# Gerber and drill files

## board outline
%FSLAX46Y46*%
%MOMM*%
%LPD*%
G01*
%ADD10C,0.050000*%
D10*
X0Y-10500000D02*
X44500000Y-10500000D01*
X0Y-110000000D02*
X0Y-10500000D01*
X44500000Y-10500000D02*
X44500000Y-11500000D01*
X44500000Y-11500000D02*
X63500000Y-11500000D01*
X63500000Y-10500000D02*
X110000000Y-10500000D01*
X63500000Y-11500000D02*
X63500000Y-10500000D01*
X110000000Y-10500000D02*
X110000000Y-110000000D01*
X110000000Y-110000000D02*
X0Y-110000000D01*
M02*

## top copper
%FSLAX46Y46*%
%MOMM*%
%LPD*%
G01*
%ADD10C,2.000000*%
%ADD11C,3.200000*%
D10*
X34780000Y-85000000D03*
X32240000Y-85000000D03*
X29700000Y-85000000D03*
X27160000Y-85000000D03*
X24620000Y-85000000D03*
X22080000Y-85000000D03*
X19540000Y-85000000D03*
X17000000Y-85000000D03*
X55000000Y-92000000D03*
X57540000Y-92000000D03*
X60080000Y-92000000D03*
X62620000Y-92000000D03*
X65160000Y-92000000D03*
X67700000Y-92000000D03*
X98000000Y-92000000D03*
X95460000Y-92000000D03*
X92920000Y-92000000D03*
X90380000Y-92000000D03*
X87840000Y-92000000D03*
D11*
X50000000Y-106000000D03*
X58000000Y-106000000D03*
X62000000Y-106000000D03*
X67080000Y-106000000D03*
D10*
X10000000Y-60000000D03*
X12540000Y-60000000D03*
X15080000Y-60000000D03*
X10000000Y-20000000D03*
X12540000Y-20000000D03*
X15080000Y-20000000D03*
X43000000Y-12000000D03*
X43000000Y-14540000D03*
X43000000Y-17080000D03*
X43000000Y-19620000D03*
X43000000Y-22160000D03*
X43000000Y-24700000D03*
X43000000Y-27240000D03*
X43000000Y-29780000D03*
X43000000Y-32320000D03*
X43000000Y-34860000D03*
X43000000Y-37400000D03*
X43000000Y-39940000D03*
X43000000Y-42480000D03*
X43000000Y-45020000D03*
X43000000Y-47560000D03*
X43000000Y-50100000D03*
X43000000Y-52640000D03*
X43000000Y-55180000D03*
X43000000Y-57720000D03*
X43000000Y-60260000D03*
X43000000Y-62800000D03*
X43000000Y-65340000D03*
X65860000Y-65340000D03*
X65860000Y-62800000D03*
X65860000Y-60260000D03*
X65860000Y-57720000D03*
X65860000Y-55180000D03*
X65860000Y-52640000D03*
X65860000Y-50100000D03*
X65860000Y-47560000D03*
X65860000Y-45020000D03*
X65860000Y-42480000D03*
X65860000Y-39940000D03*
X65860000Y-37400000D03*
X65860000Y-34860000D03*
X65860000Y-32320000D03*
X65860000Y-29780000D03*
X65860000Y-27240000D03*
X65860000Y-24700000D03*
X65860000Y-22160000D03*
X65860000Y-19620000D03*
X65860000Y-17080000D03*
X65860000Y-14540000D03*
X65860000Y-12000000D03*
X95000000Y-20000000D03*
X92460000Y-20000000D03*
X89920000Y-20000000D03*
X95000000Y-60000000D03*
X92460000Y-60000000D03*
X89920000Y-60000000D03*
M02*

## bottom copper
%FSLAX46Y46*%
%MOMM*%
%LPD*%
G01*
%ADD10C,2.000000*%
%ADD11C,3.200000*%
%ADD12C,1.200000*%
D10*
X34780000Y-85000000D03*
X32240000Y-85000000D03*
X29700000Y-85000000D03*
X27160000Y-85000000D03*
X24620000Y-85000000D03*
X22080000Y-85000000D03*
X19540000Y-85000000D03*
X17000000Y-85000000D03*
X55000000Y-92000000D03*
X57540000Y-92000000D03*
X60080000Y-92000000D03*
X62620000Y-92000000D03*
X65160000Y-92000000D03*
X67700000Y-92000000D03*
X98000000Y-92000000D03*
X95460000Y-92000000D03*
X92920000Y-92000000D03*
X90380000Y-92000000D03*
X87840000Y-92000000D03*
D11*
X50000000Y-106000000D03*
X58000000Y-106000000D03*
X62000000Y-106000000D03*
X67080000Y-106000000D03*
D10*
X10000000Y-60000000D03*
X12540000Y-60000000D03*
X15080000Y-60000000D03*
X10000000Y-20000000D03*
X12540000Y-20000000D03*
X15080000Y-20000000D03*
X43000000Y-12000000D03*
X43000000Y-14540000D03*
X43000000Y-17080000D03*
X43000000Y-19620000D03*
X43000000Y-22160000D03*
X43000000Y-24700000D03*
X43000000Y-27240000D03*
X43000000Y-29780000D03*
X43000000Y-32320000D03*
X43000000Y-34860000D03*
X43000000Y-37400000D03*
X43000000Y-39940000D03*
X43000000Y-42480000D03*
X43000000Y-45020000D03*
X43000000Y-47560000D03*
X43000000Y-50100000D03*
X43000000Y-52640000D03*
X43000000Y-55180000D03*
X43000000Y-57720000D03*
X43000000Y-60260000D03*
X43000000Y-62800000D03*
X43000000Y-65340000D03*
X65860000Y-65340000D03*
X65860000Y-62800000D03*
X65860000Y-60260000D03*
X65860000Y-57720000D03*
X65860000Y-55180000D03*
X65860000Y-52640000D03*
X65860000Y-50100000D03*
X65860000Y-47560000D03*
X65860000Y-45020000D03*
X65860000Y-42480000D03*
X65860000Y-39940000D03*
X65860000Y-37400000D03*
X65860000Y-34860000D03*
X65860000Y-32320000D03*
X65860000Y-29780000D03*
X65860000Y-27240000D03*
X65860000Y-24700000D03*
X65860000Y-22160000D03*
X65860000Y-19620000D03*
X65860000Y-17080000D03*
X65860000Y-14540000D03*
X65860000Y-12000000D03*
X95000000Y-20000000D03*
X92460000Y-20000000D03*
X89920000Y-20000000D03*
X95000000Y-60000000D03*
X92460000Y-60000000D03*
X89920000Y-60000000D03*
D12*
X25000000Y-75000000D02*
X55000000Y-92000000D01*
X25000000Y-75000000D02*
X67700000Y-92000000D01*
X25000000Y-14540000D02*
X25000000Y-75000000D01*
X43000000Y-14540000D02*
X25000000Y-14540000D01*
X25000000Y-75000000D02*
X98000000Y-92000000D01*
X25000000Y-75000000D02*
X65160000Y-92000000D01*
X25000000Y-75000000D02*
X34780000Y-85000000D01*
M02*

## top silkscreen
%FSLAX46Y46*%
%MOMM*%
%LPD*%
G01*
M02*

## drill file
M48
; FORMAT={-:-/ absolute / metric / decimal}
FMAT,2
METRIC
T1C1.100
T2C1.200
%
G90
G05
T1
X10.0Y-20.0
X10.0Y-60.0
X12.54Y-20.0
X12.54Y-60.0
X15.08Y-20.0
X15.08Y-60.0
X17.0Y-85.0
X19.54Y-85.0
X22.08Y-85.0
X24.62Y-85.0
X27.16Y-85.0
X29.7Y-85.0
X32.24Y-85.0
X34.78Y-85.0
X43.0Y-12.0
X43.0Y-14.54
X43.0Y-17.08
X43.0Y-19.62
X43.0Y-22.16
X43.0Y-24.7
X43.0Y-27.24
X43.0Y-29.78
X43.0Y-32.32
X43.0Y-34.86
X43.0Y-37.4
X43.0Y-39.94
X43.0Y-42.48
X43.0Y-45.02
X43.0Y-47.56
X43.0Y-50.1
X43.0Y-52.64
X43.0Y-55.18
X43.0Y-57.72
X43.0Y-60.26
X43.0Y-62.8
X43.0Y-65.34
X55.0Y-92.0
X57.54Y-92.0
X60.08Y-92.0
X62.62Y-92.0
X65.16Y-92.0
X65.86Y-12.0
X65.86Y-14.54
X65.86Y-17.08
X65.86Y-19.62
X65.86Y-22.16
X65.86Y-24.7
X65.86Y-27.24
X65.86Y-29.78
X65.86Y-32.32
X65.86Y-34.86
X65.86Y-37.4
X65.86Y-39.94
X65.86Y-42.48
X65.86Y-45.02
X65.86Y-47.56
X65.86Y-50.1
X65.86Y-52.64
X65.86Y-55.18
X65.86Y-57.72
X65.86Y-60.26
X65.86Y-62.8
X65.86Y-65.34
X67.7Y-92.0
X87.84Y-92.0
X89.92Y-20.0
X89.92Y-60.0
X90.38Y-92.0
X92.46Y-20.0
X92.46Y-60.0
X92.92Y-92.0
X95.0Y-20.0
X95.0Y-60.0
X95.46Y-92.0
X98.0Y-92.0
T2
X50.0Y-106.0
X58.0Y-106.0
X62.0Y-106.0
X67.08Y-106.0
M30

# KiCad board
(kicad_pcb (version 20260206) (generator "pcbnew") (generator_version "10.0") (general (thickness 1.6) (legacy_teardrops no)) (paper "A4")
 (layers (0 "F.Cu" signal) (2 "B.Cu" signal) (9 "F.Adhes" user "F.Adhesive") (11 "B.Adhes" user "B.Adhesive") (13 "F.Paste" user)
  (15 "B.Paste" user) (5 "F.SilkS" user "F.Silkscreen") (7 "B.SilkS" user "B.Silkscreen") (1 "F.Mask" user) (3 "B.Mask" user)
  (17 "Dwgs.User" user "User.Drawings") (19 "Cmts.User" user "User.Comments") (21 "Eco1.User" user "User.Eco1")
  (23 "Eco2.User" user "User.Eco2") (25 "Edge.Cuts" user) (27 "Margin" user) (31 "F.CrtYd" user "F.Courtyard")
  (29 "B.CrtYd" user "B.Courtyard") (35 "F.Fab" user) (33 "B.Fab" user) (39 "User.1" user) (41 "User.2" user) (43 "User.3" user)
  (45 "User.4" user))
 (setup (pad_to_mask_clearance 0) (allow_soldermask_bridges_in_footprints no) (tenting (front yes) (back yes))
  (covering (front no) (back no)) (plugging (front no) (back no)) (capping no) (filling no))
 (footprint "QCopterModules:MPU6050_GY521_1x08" (layer "F.Cu") (at 34.78 85 -90)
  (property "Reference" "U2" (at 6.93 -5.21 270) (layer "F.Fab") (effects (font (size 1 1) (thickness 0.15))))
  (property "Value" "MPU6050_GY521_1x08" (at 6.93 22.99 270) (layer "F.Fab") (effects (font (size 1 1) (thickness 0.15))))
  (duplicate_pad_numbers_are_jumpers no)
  (pad "1" thru_hole circle (at 0 0 270) (size 2 2) (drill 1.1) (layers "*.Cu" "*.Mask") (remove_unused_layers no) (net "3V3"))
  (pad "2" thru_hole circle (at 0 2.54 270) (size 2 2) (drill 1.1) (layers "*.Cu" "*.Mask") (remove_unused_layers no) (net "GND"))
  (pad "3" thru_hole circle (at 0 5.08 270) (size 2 2) (drill 1.1) (layers "*.Cu" "*.Mask") (remove_unused_layers no) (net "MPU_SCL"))
  (pad "4" thru_hole circle (at 0 7.62 270) (size 2 2) (drill 1.1) (layers "*.Cu" "*.Mask") (remove_unused_layers no) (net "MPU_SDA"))
  (pad "5" thru_hole circle (at 0 10.16 270) (size 2 2) (drill 1.1) (layers "*.Cu" "*.Mask") (remove_unused_layers no)
   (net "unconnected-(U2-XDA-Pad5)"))
  (pad "6" thru_hole circle (at 0 12.7 270) (size 2 2) (drill 1.1) (layers "*.Cu" "*.Mask") (remove_unused_layers no)
   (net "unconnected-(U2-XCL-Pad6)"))
  (pad "7" thru_hole circle (at 0 15.24 270) (size 2 2) (drill 1.1) (layers "*.Cu" "*.Mask") (remove_unused_layers no) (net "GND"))
  (pad "8" thru_hole circle (at 0 17.78 270) (size 2 2) (drill 1.1) (layers "*.Cu" "*.Mask") (remove_unused_layers no) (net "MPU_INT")))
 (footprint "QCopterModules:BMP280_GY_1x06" (layer "F.Cu") (at 55 92 90)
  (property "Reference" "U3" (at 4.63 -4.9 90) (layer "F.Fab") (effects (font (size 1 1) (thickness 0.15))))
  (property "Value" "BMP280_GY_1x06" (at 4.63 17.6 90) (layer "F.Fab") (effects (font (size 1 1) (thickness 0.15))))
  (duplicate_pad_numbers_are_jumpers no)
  (pad "1" thru_hole circle (at 0 0 90) (size 2 2) (drill 1.1) (layers "*.Cu" "*.Mask") (remove_unused_layers no) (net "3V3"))
  (pad "2" thru_hole circle (at 0 2.54 90) (size 2 2) (drill 1.1) (layers "*.Cu" "*.Mask") (remove_unused_layers no) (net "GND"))
  (pad "3" thru_hole circle (at 0 5.08 90) (size 2 2) (drill 1.1) (layers "*.Cu" "*.Mask") (remove_unused_layers no) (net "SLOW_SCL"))
  (pad "4" thru_hole circle (at 0 7.62 90) (size 2 2) (drill 1.1) (layers "*.Cu" "*.Mask") (remove_unused_layers no) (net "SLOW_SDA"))
  (pad "5" thru_hole circle (at 0 10.16 90) (size 2 2) (drill 1.1) (layers "*.Cu" "*.Mask") (remove_unused_layers no) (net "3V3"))
  (pad "6" thru_hole circle (at 0 12.7 90) (size 2 2) (drill 1.1) (layers "*.Cu" "*.Mask") (remove_unused_layers no) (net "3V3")))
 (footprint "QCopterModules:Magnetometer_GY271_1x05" (layer "F.Cu") (at 98 92 -90)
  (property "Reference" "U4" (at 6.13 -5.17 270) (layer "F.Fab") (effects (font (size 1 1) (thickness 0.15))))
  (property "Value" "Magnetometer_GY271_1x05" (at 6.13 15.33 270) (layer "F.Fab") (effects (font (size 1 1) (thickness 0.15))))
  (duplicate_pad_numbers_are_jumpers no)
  (pad "1" thru_hole circle (at 0 0 270) (size 2 2) (drill 1.1) (layers "*.Cu" "*.Mask") (remove_unused_layers no) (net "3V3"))
  (pad "2" thru_hole circle (at 0 2.54 270) (size 2 2) (drill 1.1) (layers "*.Cu" "*.Mask") (remove_unused_layers no) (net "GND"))
  (pad "3" thru_hole circle (at 0 5.08 270) (size 2 2) (drill 1.1) (layers "*.Cu" "*.Mask") (remove_unused_layers no) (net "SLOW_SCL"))
  (pad "4" thru_hole circle (at 0 7.62 270) (size 2 2) (drill 1.1) (layers "*.Cu" "*.Mask") (remove_unused_layers no) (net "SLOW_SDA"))
  (pad "5" thru_hole circle (at 0 10.16 270) (size 2 2) (drill 1.1) (layers "*.Cu" "*.Mask") (remove_unused_layers no) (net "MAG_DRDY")))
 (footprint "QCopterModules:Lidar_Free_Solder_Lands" (layer "F.Cu") (at 50 106)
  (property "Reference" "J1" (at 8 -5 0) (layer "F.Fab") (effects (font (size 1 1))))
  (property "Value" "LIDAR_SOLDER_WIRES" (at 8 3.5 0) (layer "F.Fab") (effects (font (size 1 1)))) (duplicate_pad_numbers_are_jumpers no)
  (pad "1" thru_hole circle (at 0 0) (size 3.2 3.2) (drill 1.2) (layers "*.Cu" "*.Mask") (remove_unused_layers no) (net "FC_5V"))
  (pad "2" thru_hole circle (at 8 0) (size 3.2 3.2) (drill 1.2) (layers "*.Cu" "*.Mask") (remove_unused_layers no) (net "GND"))
  (pad "3" thru_hole circle (at 12 0) (size 3.2 3.2) (drill 1.2) (layers "*.Cu" "*.Mask") (remove_unused_layers no) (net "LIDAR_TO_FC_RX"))
  (pad "4" thru_hole circle (at 17.08 0) (size 3.2 3.2) (drill 1.2) (layers "*.Cu" "*.Mask") (remove_unused_layers no)
   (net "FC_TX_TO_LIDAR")))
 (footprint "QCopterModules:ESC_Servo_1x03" (layer "F.Cu") (at 10 60 90)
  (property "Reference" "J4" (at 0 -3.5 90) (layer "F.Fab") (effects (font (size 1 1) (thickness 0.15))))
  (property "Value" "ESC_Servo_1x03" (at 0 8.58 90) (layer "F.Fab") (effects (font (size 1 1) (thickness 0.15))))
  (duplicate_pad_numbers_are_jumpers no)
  (pad "1" thru_hole circle (at 0 0 90) (size 2 2) (drill 1.1) (layers "*.Cu" "*.Mask") (remove_unused_layers no) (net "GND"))
  (pad "2" thru_hole circle (at 0 2.54 90) (size 2 2) (drill 1.1) (layers "*.Cu" "*.Mask") (remove_unused_layers no) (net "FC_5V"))
  (pad "3" thru_hole circle (at 0 5.08 90) (size 2 2) (drill 1.1) (layers "*.Cu" "*.Mask") (remove_unused_layers no) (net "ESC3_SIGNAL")))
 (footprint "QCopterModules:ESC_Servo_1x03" (layer "F.Cu") (at 10 20 90)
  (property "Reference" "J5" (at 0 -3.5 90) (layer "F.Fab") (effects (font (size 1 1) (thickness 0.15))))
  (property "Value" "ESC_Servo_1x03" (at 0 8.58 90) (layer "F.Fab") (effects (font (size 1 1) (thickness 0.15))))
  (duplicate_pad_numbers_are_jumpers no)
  (pad "1" thru_hole circle (at 0 0 90) (size 2 2) (drill 1.1) (layers "*.Cu" "*.Mask") (remove_unused_layers no) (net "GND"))
  (pad "2" thru_hole circle (at 0 2.54 90) (size 2 2) (drill 1.1) (layers "*.Cu" "*.Mask") (remove_unused_layers no)
   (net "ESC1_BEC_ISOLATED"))
  (pad "3" thru_hole circle (at 0 5.08 90) (size 2 2) (drill 1.1) (layers "*.Cu" "*.Mask") (remove_unused_layers no) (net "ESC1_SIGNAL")))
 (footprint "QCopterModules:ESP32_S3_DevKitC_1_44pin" (layer "F.Cu") (at 43 12)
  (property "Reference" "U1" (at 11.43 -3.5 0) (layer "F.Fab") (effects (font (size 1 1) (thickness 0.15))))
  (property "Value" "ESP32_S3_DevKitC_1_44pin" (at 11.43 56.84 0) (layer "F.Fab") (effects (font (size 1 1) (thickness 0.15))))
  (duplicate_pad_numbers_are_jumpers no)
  (pad "1" thru_hole circle (at 0 0) (size 2 2) (drill 1.1) (layers "*.Cu" "*.Mask") (remove_unused_layers no))
  (pad "2" thru_hole circle (at 0 2.54) (size 2 2) (drill 1.1) (layers "*.Cu" "*.Mask") (remove_unused_layers no) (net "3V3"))
  (pad "3" thru_hole circle (at 0 5.08) (size 2 2) (drill 1.1) (layers "*.Cu" "*.Mask") (remove_unused_layers no)
   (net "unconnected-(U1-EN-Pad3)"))
  (pad "4" thru_hole circle (at 0 7.62) (size 2 2) (drill 1.1) (layers "*.Cu" "*.Mask") (remove_unused_layers no) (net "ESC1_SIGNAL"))
  (pad "5" thru_hole circle (at 0 10.16) (size 2 2) (drill 1.1) (layers "*.Cu" "*.Mask") (remove_unused_layers no)
   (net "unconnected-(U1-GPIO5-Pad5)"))
  (pad "6" thru_hole circle (at 0 12.7) (size 2 2) (drill 1.1) (layers "*.Cu" "*.Mask") (remove_unused_layers no)
   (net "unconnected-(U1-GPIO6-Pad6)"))
  (pad "7" thru_hole circle (at 0 15.24) (size 2 2) (drill 1.1) (layers "*.Cu" "*.Mask") (remove_unused_layers no)
   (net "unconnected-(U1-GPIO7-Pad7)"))
  (pad "8" thru_hole circle (at 0 17.78) (size 2 2) (drill 1.1) (layers "*.Cu" "*.Mask") (remove_unused_layers no) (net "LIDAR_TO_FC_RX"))
  (pad "9" thru_hole circle (at 0 20.32) (size 2 2) (drill 1.1) (layers "*.Cu" "*.Mask") (remove_unused_layers no) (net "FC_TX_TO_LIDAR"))
  (pad "10" thru_hole circle (at 0 22.86) (size 2 2) (drill 1.1) (layers "*.Cu" "*.Mask") (remove_unused_layers no)
   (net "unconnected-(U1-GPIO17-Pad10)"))
  (pad "11" thru_hole circle (at 0 25.4) (size 2 2) (drill 1.1) (layers "*.Cu" "*.Mask") (remove_unused_layers no) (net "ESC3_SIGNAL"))
  (pad "12" thru_hole circle (at 0 27.94) (size 2 2) (drill 1.1) (layers "*.Cu" "*.Mask") (remove_unused_layers no)
   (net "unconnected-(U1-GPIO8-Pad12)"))
  (pad "13" thru_hole circle (at 0 30.48) (size 2 2) (drill 1.1) (layers "*.Cu" "*.Mask") (remove_unused_layers no)
   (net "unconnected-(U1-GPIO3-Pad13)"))
  (pad "14" thru_hole circle (at 0 33.02) (size 2 2) (drill 1.1) (layers "*.Cu" "*.Mask") (remove_unused_layers no)
   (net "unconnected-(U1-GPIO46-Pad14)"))
  (pad "15" thru_hole circle (at 0 35.56) (size 2 2) (drill 1.1) (layers "*.Cu" "*.Mask") (remove_unused_layers no)
   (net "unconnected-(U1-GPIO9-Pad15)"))
  (pad "16" thru_hole circle (at 0 38.1) (size 2 2) (drill 1.1) (layers "*.Cu" "*.Mask") (remove_unused_layers no)
   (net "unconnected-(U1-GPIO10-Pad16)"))
  (pad "17" thru_hole circle (at 0 40.64) (size 2 2) (drill 1.1) (layers "*.Cu" "*.Mask") (remove_unused_layers no)
   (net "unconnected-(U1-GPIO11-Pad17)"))
  (pad "18" thru_hole circle (at 0 43.18) (size 2 2) (drill 1.1) (layers "*.Cu" "*.Mask") (remove_unused_layers no) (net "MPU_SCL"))
  (pad "19" thru_hole circle (at 0 45.72) (size 2 2) (drill 1.1) (layers "*.Cu" "*.Mask") (remove_unused_layers no) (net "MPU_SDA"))
  (pad "20" thru_hole circle (at 0 48.26) (size 2 2) (drill 1.1) (layers "*.Cu" "*.Mask") (remove_unused_layers no) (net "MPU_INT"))
  (pad "21" thru_hole circle (at 0 50.8) (size 2 2) (drill 1.1) (layers "*.Cu" "*.Mask") (remove_unused_layers no) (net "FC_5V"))
  (pad "22" thru_hole circle (at 0 53.34) (size 2 2) (drill 1.1) (layers "*.Cu" "*.Mask") (remove_unused_layers no) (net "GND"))
  (pad "23" thru_hole circle (at 22.86 53.34) (size 2 2) (drill 1.1) (layers "*.Cu" "*.Mask") (remove_unused_layers no) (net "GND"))
  (pad "24" thru_hole circle (at 22.86 50.8) (size 2 2) (drill 1.1) (layers "*.Cu" "*.Mask") (remove_unused_layers no) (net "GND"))
  (pad "25" thru_hole circle (at 22.86 48.26) (size 2 2) (drill 1.1) (layers "*.Cu" "*.Mask") (remove_unused_layers no)
   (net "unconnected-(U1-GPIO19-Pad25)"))
  (pad "26" thru_hole circle (at 22.86 45.72) (size 2 2) (drill 1.1) (layers "*.Cu" "*.Mask") (remove_unused_layers no)
   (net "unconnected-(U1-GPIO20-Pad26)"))
  (pad "27" thru_hole circle (at 22.86 43.18) (size 2 2) (drill 1.1) (layers "*.Cu" "*.Mask") (remove_unused_layers no) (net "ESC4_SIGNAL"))
  (pad "28" thru_hole circle (at 22.86 40.64) (size 2 2) (drill 1.1) (layers "*.Cu" "*.Mask") (remove_unused_layers no)
   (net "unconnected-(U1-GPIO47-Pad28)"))
  (pad "29" thru_hole circle (at 22.86 38.1) (size 2 2) (drill 1.1) (layers "*.Cu" "*.Mask") (remove_unused_layers no)
   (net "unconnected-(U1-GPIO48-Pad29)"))
  (pad "30" thru_hole circle (at 22.86 35.56) (size 2 2) (drill 1.1) (layers "*.Cu" "*.Mask") (remove_unused_layers no)
   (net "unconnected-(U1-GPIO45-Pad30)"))
  (pad "31" thru_hole circle (at 22.86 33.02) (size 2 2) (drill 1.1) (layers "*.Cu" "*.Mask") (remove_unused_layers no)
   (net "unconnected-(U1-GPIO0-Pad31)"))
  (pad "32" thru_hole circle (at 22.86 30.48) (size 2 2) (drill 1.1) (layers "*.Cu" "*.Mask") (remove_unused_layers no)
   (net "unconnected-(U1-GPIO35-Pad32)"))
  (pad "33" thru_hole circle (at 22.86 27.94) (size 2 2) (drill 1.1) (layers "*.Cu" "*.Mask") (remove_unused_layers no)
   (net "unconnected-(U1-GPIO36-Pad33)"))
  (pad "34" thru_hole circle (at 22.86 25.4) (size 2 2) (drill 1.1) (layers "*.Cu" "*.Mask") (remove_unused_layers no)
   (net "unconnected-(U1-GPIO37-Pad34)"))
  (pad "35" thru_hole circle (at 22.86 22.86) (size 2 2) (drill 1.1) (layers "*.Cu" "*.Mask") (remove_unused_layers no)
   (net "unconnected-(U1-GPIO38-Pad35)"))
  (pad "36" thru_hole circle (at 22.86 20.32) (size 2 2) (drill 1.1) (layers "*.Cu" "*.Mask") (remove_unused_layers no) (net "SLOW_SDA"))
  (pad "37" thru_hole circle (at 22.86 17.78) (size 2 2) (drill 1.1) (layers "*.Cu" "*.Mask") (remove_unused_layers no) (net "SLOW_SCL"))
  (pad "38" thru_hole circle (at 22.86 15.24) (size 2 2) (drill 1.1) (layers "*.Cu" "*.Mask") (remove_unused_layers no) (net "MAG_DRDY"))
  (pad "39" thru_hole circle (at 22.86 12.7) (size 2 2) (drill 1.1) (layers "*.Cu" "*.Mask") (remove_unused_layers no)
   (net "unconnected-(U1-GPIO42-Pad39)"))
  (pad "40" thru_hole circle (at 22.86 10.16) (size 2 2) (drill 1.1) (layers "*.Cu" "*.Mask") (remove_unused_layers no) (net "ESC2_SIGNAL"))
  (pad "41" thru_hole circle (at 22.86 7.62) (size 2 2) (drill 1.1) (layers "*.Cu" "*.Mask") (remove_unused_layers no)
   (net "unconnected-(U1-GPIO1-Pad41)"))
  (pad "42" thru_hole circle (at 22.86 5.08) (size 2 2) (drill 1.1) (layers "*.Cu" "*.Mask") (remove_unused_layers no)
   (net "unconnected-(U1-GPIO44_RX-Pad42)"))
  (pad "43" thru_hole circle (at 22.86 2.54) (size 2 2) (drill 1.1) (layers "*.Cu" "*.Mask") (remove_unused_layers no)
   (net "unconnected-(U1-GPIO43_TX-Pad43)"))
  (pad "44" thru_hole circle (at 22.86 0) (size 2 2) (drill 1.1) (layers "*.Cu" "*.Mask") (remove_unused_layers no) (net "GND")))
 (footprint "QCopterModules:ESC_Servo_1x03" (layer "F.Cu") (at 95 20 -90)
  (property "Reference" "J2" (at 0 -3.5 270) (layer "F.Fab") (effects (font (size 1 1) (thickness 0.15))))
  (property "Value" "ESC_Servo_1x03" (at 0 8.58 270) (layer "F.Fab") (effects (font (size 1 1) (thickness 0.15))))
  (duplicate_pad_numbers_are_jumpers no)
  (pad "1" thru_hole circle (at 0 0 270) (size 2 2) (drill 1.1) (layers "*.Cu" "*.Mask") (remove_unused_layers no) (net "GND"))
  (pad "2" thru_hole circle (at 0 2.54 270) (size 2 2) (drill 1.1) (layers "*.Cu" "*.Mask") (remove_unused_layers no)
   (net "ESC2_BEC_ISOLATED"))
  (pad "3" thru_hole circle (at 0 5.08 270) (size 2 2) (drill 1.1) (layers "*.Cu" "*.Mask") (remove_unused_layers no) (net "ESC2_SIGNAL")))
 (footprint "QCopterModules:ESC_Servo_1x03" (layer "F.Cu") (at 95 60 -90)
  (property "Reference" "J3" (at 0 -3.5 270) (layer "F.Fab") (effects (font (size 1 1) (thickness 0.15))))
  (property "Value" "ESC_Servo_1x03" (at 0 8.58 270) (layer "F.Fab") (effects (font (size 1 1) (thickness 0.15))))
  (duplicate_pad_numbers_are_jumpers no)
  (pad "1" thru_hole circle (at 0 0 270) (size 2 2) (drill 1.1) (layers "*.Cu" "*.Mask") (remove_unused_layers no) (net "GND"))
  (pad "2" thru_hole circle (at 0 2.54 270) (size 2 2) (drill 1.1) (layers "*.Cu" "*.Mask") (remove_unused_layers no)
   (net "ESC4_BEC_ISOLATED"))
  (pad "3" thru_hole circle (at 0 5.08 270) (size 2 2) (drill 1.1) (layers "*.Cu" "*.Mask") (remove_unused_layers no) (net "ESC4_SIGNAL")))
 (gr_line (start 0 10.5) (end 44.5 10.5) (stroke (width 0.05) (type default)) (layer "Edge.Cuts"))
 (gr_line (start 0 110) (end 0 10.5) (stroke (width 0.05) (type default)) (layer "Edge.Cuts"))
 (gr_line (start 44.5 10.5) (end 44.5 11.5) (stroke (width 0.05) (type default)) (layer "Edge.Cuts"))
 (gr_line (start 44.5 11.5) (end 63.5 11.5) (stroke (width 0.05) (type default)) (layer "Edge.Cuts"))
 (gr_line (start 63.5 10.5) (end 110 10.5) (stroke (width 0.05) (type default)) (layer "Edge.Cuts"))
 (gr_line (start 63.5 11.5) (end 63.5 10.5) (stroke (width 0.05) (type default)) (layer "Edge.Cuts"))
 (gr_line (start 110 10.5) (end 110 110) (stroke (width 0.05) (type default)) (layer "Edge.Cuts"))
 (gr_line (start 110 110) (end 0 110) (stroke (width 0.05) (type default)) (layer "Edge.Cuts"))
 (segment (start 25 75) (end 55 92) (width 1.2) (layer "B.Cu") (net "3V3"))
 (segment (start 25 75) (end 67.7 92) (width 1.2) (layer "B.Cu") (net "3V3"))
 (segment (start 25 14.54) (end 25 75) (width 1.2) (layer "B.Cu") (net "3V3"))
 (segment (start 43 14.54) (end 25 14.54) (width 1.2) (layer "B.Cu") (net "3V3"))
 (segment (start 25 75) (end 98 92) (width 1.2) (layer "B.Cu") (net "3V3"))
 (segment (start 25 75) (end 65.16 92) (width 1.2) (layer "B.Cu") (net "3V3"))
 (segment (start 25 75) (end 34.78 85) (width 1.2) (layer "B.Cu") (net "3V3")))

